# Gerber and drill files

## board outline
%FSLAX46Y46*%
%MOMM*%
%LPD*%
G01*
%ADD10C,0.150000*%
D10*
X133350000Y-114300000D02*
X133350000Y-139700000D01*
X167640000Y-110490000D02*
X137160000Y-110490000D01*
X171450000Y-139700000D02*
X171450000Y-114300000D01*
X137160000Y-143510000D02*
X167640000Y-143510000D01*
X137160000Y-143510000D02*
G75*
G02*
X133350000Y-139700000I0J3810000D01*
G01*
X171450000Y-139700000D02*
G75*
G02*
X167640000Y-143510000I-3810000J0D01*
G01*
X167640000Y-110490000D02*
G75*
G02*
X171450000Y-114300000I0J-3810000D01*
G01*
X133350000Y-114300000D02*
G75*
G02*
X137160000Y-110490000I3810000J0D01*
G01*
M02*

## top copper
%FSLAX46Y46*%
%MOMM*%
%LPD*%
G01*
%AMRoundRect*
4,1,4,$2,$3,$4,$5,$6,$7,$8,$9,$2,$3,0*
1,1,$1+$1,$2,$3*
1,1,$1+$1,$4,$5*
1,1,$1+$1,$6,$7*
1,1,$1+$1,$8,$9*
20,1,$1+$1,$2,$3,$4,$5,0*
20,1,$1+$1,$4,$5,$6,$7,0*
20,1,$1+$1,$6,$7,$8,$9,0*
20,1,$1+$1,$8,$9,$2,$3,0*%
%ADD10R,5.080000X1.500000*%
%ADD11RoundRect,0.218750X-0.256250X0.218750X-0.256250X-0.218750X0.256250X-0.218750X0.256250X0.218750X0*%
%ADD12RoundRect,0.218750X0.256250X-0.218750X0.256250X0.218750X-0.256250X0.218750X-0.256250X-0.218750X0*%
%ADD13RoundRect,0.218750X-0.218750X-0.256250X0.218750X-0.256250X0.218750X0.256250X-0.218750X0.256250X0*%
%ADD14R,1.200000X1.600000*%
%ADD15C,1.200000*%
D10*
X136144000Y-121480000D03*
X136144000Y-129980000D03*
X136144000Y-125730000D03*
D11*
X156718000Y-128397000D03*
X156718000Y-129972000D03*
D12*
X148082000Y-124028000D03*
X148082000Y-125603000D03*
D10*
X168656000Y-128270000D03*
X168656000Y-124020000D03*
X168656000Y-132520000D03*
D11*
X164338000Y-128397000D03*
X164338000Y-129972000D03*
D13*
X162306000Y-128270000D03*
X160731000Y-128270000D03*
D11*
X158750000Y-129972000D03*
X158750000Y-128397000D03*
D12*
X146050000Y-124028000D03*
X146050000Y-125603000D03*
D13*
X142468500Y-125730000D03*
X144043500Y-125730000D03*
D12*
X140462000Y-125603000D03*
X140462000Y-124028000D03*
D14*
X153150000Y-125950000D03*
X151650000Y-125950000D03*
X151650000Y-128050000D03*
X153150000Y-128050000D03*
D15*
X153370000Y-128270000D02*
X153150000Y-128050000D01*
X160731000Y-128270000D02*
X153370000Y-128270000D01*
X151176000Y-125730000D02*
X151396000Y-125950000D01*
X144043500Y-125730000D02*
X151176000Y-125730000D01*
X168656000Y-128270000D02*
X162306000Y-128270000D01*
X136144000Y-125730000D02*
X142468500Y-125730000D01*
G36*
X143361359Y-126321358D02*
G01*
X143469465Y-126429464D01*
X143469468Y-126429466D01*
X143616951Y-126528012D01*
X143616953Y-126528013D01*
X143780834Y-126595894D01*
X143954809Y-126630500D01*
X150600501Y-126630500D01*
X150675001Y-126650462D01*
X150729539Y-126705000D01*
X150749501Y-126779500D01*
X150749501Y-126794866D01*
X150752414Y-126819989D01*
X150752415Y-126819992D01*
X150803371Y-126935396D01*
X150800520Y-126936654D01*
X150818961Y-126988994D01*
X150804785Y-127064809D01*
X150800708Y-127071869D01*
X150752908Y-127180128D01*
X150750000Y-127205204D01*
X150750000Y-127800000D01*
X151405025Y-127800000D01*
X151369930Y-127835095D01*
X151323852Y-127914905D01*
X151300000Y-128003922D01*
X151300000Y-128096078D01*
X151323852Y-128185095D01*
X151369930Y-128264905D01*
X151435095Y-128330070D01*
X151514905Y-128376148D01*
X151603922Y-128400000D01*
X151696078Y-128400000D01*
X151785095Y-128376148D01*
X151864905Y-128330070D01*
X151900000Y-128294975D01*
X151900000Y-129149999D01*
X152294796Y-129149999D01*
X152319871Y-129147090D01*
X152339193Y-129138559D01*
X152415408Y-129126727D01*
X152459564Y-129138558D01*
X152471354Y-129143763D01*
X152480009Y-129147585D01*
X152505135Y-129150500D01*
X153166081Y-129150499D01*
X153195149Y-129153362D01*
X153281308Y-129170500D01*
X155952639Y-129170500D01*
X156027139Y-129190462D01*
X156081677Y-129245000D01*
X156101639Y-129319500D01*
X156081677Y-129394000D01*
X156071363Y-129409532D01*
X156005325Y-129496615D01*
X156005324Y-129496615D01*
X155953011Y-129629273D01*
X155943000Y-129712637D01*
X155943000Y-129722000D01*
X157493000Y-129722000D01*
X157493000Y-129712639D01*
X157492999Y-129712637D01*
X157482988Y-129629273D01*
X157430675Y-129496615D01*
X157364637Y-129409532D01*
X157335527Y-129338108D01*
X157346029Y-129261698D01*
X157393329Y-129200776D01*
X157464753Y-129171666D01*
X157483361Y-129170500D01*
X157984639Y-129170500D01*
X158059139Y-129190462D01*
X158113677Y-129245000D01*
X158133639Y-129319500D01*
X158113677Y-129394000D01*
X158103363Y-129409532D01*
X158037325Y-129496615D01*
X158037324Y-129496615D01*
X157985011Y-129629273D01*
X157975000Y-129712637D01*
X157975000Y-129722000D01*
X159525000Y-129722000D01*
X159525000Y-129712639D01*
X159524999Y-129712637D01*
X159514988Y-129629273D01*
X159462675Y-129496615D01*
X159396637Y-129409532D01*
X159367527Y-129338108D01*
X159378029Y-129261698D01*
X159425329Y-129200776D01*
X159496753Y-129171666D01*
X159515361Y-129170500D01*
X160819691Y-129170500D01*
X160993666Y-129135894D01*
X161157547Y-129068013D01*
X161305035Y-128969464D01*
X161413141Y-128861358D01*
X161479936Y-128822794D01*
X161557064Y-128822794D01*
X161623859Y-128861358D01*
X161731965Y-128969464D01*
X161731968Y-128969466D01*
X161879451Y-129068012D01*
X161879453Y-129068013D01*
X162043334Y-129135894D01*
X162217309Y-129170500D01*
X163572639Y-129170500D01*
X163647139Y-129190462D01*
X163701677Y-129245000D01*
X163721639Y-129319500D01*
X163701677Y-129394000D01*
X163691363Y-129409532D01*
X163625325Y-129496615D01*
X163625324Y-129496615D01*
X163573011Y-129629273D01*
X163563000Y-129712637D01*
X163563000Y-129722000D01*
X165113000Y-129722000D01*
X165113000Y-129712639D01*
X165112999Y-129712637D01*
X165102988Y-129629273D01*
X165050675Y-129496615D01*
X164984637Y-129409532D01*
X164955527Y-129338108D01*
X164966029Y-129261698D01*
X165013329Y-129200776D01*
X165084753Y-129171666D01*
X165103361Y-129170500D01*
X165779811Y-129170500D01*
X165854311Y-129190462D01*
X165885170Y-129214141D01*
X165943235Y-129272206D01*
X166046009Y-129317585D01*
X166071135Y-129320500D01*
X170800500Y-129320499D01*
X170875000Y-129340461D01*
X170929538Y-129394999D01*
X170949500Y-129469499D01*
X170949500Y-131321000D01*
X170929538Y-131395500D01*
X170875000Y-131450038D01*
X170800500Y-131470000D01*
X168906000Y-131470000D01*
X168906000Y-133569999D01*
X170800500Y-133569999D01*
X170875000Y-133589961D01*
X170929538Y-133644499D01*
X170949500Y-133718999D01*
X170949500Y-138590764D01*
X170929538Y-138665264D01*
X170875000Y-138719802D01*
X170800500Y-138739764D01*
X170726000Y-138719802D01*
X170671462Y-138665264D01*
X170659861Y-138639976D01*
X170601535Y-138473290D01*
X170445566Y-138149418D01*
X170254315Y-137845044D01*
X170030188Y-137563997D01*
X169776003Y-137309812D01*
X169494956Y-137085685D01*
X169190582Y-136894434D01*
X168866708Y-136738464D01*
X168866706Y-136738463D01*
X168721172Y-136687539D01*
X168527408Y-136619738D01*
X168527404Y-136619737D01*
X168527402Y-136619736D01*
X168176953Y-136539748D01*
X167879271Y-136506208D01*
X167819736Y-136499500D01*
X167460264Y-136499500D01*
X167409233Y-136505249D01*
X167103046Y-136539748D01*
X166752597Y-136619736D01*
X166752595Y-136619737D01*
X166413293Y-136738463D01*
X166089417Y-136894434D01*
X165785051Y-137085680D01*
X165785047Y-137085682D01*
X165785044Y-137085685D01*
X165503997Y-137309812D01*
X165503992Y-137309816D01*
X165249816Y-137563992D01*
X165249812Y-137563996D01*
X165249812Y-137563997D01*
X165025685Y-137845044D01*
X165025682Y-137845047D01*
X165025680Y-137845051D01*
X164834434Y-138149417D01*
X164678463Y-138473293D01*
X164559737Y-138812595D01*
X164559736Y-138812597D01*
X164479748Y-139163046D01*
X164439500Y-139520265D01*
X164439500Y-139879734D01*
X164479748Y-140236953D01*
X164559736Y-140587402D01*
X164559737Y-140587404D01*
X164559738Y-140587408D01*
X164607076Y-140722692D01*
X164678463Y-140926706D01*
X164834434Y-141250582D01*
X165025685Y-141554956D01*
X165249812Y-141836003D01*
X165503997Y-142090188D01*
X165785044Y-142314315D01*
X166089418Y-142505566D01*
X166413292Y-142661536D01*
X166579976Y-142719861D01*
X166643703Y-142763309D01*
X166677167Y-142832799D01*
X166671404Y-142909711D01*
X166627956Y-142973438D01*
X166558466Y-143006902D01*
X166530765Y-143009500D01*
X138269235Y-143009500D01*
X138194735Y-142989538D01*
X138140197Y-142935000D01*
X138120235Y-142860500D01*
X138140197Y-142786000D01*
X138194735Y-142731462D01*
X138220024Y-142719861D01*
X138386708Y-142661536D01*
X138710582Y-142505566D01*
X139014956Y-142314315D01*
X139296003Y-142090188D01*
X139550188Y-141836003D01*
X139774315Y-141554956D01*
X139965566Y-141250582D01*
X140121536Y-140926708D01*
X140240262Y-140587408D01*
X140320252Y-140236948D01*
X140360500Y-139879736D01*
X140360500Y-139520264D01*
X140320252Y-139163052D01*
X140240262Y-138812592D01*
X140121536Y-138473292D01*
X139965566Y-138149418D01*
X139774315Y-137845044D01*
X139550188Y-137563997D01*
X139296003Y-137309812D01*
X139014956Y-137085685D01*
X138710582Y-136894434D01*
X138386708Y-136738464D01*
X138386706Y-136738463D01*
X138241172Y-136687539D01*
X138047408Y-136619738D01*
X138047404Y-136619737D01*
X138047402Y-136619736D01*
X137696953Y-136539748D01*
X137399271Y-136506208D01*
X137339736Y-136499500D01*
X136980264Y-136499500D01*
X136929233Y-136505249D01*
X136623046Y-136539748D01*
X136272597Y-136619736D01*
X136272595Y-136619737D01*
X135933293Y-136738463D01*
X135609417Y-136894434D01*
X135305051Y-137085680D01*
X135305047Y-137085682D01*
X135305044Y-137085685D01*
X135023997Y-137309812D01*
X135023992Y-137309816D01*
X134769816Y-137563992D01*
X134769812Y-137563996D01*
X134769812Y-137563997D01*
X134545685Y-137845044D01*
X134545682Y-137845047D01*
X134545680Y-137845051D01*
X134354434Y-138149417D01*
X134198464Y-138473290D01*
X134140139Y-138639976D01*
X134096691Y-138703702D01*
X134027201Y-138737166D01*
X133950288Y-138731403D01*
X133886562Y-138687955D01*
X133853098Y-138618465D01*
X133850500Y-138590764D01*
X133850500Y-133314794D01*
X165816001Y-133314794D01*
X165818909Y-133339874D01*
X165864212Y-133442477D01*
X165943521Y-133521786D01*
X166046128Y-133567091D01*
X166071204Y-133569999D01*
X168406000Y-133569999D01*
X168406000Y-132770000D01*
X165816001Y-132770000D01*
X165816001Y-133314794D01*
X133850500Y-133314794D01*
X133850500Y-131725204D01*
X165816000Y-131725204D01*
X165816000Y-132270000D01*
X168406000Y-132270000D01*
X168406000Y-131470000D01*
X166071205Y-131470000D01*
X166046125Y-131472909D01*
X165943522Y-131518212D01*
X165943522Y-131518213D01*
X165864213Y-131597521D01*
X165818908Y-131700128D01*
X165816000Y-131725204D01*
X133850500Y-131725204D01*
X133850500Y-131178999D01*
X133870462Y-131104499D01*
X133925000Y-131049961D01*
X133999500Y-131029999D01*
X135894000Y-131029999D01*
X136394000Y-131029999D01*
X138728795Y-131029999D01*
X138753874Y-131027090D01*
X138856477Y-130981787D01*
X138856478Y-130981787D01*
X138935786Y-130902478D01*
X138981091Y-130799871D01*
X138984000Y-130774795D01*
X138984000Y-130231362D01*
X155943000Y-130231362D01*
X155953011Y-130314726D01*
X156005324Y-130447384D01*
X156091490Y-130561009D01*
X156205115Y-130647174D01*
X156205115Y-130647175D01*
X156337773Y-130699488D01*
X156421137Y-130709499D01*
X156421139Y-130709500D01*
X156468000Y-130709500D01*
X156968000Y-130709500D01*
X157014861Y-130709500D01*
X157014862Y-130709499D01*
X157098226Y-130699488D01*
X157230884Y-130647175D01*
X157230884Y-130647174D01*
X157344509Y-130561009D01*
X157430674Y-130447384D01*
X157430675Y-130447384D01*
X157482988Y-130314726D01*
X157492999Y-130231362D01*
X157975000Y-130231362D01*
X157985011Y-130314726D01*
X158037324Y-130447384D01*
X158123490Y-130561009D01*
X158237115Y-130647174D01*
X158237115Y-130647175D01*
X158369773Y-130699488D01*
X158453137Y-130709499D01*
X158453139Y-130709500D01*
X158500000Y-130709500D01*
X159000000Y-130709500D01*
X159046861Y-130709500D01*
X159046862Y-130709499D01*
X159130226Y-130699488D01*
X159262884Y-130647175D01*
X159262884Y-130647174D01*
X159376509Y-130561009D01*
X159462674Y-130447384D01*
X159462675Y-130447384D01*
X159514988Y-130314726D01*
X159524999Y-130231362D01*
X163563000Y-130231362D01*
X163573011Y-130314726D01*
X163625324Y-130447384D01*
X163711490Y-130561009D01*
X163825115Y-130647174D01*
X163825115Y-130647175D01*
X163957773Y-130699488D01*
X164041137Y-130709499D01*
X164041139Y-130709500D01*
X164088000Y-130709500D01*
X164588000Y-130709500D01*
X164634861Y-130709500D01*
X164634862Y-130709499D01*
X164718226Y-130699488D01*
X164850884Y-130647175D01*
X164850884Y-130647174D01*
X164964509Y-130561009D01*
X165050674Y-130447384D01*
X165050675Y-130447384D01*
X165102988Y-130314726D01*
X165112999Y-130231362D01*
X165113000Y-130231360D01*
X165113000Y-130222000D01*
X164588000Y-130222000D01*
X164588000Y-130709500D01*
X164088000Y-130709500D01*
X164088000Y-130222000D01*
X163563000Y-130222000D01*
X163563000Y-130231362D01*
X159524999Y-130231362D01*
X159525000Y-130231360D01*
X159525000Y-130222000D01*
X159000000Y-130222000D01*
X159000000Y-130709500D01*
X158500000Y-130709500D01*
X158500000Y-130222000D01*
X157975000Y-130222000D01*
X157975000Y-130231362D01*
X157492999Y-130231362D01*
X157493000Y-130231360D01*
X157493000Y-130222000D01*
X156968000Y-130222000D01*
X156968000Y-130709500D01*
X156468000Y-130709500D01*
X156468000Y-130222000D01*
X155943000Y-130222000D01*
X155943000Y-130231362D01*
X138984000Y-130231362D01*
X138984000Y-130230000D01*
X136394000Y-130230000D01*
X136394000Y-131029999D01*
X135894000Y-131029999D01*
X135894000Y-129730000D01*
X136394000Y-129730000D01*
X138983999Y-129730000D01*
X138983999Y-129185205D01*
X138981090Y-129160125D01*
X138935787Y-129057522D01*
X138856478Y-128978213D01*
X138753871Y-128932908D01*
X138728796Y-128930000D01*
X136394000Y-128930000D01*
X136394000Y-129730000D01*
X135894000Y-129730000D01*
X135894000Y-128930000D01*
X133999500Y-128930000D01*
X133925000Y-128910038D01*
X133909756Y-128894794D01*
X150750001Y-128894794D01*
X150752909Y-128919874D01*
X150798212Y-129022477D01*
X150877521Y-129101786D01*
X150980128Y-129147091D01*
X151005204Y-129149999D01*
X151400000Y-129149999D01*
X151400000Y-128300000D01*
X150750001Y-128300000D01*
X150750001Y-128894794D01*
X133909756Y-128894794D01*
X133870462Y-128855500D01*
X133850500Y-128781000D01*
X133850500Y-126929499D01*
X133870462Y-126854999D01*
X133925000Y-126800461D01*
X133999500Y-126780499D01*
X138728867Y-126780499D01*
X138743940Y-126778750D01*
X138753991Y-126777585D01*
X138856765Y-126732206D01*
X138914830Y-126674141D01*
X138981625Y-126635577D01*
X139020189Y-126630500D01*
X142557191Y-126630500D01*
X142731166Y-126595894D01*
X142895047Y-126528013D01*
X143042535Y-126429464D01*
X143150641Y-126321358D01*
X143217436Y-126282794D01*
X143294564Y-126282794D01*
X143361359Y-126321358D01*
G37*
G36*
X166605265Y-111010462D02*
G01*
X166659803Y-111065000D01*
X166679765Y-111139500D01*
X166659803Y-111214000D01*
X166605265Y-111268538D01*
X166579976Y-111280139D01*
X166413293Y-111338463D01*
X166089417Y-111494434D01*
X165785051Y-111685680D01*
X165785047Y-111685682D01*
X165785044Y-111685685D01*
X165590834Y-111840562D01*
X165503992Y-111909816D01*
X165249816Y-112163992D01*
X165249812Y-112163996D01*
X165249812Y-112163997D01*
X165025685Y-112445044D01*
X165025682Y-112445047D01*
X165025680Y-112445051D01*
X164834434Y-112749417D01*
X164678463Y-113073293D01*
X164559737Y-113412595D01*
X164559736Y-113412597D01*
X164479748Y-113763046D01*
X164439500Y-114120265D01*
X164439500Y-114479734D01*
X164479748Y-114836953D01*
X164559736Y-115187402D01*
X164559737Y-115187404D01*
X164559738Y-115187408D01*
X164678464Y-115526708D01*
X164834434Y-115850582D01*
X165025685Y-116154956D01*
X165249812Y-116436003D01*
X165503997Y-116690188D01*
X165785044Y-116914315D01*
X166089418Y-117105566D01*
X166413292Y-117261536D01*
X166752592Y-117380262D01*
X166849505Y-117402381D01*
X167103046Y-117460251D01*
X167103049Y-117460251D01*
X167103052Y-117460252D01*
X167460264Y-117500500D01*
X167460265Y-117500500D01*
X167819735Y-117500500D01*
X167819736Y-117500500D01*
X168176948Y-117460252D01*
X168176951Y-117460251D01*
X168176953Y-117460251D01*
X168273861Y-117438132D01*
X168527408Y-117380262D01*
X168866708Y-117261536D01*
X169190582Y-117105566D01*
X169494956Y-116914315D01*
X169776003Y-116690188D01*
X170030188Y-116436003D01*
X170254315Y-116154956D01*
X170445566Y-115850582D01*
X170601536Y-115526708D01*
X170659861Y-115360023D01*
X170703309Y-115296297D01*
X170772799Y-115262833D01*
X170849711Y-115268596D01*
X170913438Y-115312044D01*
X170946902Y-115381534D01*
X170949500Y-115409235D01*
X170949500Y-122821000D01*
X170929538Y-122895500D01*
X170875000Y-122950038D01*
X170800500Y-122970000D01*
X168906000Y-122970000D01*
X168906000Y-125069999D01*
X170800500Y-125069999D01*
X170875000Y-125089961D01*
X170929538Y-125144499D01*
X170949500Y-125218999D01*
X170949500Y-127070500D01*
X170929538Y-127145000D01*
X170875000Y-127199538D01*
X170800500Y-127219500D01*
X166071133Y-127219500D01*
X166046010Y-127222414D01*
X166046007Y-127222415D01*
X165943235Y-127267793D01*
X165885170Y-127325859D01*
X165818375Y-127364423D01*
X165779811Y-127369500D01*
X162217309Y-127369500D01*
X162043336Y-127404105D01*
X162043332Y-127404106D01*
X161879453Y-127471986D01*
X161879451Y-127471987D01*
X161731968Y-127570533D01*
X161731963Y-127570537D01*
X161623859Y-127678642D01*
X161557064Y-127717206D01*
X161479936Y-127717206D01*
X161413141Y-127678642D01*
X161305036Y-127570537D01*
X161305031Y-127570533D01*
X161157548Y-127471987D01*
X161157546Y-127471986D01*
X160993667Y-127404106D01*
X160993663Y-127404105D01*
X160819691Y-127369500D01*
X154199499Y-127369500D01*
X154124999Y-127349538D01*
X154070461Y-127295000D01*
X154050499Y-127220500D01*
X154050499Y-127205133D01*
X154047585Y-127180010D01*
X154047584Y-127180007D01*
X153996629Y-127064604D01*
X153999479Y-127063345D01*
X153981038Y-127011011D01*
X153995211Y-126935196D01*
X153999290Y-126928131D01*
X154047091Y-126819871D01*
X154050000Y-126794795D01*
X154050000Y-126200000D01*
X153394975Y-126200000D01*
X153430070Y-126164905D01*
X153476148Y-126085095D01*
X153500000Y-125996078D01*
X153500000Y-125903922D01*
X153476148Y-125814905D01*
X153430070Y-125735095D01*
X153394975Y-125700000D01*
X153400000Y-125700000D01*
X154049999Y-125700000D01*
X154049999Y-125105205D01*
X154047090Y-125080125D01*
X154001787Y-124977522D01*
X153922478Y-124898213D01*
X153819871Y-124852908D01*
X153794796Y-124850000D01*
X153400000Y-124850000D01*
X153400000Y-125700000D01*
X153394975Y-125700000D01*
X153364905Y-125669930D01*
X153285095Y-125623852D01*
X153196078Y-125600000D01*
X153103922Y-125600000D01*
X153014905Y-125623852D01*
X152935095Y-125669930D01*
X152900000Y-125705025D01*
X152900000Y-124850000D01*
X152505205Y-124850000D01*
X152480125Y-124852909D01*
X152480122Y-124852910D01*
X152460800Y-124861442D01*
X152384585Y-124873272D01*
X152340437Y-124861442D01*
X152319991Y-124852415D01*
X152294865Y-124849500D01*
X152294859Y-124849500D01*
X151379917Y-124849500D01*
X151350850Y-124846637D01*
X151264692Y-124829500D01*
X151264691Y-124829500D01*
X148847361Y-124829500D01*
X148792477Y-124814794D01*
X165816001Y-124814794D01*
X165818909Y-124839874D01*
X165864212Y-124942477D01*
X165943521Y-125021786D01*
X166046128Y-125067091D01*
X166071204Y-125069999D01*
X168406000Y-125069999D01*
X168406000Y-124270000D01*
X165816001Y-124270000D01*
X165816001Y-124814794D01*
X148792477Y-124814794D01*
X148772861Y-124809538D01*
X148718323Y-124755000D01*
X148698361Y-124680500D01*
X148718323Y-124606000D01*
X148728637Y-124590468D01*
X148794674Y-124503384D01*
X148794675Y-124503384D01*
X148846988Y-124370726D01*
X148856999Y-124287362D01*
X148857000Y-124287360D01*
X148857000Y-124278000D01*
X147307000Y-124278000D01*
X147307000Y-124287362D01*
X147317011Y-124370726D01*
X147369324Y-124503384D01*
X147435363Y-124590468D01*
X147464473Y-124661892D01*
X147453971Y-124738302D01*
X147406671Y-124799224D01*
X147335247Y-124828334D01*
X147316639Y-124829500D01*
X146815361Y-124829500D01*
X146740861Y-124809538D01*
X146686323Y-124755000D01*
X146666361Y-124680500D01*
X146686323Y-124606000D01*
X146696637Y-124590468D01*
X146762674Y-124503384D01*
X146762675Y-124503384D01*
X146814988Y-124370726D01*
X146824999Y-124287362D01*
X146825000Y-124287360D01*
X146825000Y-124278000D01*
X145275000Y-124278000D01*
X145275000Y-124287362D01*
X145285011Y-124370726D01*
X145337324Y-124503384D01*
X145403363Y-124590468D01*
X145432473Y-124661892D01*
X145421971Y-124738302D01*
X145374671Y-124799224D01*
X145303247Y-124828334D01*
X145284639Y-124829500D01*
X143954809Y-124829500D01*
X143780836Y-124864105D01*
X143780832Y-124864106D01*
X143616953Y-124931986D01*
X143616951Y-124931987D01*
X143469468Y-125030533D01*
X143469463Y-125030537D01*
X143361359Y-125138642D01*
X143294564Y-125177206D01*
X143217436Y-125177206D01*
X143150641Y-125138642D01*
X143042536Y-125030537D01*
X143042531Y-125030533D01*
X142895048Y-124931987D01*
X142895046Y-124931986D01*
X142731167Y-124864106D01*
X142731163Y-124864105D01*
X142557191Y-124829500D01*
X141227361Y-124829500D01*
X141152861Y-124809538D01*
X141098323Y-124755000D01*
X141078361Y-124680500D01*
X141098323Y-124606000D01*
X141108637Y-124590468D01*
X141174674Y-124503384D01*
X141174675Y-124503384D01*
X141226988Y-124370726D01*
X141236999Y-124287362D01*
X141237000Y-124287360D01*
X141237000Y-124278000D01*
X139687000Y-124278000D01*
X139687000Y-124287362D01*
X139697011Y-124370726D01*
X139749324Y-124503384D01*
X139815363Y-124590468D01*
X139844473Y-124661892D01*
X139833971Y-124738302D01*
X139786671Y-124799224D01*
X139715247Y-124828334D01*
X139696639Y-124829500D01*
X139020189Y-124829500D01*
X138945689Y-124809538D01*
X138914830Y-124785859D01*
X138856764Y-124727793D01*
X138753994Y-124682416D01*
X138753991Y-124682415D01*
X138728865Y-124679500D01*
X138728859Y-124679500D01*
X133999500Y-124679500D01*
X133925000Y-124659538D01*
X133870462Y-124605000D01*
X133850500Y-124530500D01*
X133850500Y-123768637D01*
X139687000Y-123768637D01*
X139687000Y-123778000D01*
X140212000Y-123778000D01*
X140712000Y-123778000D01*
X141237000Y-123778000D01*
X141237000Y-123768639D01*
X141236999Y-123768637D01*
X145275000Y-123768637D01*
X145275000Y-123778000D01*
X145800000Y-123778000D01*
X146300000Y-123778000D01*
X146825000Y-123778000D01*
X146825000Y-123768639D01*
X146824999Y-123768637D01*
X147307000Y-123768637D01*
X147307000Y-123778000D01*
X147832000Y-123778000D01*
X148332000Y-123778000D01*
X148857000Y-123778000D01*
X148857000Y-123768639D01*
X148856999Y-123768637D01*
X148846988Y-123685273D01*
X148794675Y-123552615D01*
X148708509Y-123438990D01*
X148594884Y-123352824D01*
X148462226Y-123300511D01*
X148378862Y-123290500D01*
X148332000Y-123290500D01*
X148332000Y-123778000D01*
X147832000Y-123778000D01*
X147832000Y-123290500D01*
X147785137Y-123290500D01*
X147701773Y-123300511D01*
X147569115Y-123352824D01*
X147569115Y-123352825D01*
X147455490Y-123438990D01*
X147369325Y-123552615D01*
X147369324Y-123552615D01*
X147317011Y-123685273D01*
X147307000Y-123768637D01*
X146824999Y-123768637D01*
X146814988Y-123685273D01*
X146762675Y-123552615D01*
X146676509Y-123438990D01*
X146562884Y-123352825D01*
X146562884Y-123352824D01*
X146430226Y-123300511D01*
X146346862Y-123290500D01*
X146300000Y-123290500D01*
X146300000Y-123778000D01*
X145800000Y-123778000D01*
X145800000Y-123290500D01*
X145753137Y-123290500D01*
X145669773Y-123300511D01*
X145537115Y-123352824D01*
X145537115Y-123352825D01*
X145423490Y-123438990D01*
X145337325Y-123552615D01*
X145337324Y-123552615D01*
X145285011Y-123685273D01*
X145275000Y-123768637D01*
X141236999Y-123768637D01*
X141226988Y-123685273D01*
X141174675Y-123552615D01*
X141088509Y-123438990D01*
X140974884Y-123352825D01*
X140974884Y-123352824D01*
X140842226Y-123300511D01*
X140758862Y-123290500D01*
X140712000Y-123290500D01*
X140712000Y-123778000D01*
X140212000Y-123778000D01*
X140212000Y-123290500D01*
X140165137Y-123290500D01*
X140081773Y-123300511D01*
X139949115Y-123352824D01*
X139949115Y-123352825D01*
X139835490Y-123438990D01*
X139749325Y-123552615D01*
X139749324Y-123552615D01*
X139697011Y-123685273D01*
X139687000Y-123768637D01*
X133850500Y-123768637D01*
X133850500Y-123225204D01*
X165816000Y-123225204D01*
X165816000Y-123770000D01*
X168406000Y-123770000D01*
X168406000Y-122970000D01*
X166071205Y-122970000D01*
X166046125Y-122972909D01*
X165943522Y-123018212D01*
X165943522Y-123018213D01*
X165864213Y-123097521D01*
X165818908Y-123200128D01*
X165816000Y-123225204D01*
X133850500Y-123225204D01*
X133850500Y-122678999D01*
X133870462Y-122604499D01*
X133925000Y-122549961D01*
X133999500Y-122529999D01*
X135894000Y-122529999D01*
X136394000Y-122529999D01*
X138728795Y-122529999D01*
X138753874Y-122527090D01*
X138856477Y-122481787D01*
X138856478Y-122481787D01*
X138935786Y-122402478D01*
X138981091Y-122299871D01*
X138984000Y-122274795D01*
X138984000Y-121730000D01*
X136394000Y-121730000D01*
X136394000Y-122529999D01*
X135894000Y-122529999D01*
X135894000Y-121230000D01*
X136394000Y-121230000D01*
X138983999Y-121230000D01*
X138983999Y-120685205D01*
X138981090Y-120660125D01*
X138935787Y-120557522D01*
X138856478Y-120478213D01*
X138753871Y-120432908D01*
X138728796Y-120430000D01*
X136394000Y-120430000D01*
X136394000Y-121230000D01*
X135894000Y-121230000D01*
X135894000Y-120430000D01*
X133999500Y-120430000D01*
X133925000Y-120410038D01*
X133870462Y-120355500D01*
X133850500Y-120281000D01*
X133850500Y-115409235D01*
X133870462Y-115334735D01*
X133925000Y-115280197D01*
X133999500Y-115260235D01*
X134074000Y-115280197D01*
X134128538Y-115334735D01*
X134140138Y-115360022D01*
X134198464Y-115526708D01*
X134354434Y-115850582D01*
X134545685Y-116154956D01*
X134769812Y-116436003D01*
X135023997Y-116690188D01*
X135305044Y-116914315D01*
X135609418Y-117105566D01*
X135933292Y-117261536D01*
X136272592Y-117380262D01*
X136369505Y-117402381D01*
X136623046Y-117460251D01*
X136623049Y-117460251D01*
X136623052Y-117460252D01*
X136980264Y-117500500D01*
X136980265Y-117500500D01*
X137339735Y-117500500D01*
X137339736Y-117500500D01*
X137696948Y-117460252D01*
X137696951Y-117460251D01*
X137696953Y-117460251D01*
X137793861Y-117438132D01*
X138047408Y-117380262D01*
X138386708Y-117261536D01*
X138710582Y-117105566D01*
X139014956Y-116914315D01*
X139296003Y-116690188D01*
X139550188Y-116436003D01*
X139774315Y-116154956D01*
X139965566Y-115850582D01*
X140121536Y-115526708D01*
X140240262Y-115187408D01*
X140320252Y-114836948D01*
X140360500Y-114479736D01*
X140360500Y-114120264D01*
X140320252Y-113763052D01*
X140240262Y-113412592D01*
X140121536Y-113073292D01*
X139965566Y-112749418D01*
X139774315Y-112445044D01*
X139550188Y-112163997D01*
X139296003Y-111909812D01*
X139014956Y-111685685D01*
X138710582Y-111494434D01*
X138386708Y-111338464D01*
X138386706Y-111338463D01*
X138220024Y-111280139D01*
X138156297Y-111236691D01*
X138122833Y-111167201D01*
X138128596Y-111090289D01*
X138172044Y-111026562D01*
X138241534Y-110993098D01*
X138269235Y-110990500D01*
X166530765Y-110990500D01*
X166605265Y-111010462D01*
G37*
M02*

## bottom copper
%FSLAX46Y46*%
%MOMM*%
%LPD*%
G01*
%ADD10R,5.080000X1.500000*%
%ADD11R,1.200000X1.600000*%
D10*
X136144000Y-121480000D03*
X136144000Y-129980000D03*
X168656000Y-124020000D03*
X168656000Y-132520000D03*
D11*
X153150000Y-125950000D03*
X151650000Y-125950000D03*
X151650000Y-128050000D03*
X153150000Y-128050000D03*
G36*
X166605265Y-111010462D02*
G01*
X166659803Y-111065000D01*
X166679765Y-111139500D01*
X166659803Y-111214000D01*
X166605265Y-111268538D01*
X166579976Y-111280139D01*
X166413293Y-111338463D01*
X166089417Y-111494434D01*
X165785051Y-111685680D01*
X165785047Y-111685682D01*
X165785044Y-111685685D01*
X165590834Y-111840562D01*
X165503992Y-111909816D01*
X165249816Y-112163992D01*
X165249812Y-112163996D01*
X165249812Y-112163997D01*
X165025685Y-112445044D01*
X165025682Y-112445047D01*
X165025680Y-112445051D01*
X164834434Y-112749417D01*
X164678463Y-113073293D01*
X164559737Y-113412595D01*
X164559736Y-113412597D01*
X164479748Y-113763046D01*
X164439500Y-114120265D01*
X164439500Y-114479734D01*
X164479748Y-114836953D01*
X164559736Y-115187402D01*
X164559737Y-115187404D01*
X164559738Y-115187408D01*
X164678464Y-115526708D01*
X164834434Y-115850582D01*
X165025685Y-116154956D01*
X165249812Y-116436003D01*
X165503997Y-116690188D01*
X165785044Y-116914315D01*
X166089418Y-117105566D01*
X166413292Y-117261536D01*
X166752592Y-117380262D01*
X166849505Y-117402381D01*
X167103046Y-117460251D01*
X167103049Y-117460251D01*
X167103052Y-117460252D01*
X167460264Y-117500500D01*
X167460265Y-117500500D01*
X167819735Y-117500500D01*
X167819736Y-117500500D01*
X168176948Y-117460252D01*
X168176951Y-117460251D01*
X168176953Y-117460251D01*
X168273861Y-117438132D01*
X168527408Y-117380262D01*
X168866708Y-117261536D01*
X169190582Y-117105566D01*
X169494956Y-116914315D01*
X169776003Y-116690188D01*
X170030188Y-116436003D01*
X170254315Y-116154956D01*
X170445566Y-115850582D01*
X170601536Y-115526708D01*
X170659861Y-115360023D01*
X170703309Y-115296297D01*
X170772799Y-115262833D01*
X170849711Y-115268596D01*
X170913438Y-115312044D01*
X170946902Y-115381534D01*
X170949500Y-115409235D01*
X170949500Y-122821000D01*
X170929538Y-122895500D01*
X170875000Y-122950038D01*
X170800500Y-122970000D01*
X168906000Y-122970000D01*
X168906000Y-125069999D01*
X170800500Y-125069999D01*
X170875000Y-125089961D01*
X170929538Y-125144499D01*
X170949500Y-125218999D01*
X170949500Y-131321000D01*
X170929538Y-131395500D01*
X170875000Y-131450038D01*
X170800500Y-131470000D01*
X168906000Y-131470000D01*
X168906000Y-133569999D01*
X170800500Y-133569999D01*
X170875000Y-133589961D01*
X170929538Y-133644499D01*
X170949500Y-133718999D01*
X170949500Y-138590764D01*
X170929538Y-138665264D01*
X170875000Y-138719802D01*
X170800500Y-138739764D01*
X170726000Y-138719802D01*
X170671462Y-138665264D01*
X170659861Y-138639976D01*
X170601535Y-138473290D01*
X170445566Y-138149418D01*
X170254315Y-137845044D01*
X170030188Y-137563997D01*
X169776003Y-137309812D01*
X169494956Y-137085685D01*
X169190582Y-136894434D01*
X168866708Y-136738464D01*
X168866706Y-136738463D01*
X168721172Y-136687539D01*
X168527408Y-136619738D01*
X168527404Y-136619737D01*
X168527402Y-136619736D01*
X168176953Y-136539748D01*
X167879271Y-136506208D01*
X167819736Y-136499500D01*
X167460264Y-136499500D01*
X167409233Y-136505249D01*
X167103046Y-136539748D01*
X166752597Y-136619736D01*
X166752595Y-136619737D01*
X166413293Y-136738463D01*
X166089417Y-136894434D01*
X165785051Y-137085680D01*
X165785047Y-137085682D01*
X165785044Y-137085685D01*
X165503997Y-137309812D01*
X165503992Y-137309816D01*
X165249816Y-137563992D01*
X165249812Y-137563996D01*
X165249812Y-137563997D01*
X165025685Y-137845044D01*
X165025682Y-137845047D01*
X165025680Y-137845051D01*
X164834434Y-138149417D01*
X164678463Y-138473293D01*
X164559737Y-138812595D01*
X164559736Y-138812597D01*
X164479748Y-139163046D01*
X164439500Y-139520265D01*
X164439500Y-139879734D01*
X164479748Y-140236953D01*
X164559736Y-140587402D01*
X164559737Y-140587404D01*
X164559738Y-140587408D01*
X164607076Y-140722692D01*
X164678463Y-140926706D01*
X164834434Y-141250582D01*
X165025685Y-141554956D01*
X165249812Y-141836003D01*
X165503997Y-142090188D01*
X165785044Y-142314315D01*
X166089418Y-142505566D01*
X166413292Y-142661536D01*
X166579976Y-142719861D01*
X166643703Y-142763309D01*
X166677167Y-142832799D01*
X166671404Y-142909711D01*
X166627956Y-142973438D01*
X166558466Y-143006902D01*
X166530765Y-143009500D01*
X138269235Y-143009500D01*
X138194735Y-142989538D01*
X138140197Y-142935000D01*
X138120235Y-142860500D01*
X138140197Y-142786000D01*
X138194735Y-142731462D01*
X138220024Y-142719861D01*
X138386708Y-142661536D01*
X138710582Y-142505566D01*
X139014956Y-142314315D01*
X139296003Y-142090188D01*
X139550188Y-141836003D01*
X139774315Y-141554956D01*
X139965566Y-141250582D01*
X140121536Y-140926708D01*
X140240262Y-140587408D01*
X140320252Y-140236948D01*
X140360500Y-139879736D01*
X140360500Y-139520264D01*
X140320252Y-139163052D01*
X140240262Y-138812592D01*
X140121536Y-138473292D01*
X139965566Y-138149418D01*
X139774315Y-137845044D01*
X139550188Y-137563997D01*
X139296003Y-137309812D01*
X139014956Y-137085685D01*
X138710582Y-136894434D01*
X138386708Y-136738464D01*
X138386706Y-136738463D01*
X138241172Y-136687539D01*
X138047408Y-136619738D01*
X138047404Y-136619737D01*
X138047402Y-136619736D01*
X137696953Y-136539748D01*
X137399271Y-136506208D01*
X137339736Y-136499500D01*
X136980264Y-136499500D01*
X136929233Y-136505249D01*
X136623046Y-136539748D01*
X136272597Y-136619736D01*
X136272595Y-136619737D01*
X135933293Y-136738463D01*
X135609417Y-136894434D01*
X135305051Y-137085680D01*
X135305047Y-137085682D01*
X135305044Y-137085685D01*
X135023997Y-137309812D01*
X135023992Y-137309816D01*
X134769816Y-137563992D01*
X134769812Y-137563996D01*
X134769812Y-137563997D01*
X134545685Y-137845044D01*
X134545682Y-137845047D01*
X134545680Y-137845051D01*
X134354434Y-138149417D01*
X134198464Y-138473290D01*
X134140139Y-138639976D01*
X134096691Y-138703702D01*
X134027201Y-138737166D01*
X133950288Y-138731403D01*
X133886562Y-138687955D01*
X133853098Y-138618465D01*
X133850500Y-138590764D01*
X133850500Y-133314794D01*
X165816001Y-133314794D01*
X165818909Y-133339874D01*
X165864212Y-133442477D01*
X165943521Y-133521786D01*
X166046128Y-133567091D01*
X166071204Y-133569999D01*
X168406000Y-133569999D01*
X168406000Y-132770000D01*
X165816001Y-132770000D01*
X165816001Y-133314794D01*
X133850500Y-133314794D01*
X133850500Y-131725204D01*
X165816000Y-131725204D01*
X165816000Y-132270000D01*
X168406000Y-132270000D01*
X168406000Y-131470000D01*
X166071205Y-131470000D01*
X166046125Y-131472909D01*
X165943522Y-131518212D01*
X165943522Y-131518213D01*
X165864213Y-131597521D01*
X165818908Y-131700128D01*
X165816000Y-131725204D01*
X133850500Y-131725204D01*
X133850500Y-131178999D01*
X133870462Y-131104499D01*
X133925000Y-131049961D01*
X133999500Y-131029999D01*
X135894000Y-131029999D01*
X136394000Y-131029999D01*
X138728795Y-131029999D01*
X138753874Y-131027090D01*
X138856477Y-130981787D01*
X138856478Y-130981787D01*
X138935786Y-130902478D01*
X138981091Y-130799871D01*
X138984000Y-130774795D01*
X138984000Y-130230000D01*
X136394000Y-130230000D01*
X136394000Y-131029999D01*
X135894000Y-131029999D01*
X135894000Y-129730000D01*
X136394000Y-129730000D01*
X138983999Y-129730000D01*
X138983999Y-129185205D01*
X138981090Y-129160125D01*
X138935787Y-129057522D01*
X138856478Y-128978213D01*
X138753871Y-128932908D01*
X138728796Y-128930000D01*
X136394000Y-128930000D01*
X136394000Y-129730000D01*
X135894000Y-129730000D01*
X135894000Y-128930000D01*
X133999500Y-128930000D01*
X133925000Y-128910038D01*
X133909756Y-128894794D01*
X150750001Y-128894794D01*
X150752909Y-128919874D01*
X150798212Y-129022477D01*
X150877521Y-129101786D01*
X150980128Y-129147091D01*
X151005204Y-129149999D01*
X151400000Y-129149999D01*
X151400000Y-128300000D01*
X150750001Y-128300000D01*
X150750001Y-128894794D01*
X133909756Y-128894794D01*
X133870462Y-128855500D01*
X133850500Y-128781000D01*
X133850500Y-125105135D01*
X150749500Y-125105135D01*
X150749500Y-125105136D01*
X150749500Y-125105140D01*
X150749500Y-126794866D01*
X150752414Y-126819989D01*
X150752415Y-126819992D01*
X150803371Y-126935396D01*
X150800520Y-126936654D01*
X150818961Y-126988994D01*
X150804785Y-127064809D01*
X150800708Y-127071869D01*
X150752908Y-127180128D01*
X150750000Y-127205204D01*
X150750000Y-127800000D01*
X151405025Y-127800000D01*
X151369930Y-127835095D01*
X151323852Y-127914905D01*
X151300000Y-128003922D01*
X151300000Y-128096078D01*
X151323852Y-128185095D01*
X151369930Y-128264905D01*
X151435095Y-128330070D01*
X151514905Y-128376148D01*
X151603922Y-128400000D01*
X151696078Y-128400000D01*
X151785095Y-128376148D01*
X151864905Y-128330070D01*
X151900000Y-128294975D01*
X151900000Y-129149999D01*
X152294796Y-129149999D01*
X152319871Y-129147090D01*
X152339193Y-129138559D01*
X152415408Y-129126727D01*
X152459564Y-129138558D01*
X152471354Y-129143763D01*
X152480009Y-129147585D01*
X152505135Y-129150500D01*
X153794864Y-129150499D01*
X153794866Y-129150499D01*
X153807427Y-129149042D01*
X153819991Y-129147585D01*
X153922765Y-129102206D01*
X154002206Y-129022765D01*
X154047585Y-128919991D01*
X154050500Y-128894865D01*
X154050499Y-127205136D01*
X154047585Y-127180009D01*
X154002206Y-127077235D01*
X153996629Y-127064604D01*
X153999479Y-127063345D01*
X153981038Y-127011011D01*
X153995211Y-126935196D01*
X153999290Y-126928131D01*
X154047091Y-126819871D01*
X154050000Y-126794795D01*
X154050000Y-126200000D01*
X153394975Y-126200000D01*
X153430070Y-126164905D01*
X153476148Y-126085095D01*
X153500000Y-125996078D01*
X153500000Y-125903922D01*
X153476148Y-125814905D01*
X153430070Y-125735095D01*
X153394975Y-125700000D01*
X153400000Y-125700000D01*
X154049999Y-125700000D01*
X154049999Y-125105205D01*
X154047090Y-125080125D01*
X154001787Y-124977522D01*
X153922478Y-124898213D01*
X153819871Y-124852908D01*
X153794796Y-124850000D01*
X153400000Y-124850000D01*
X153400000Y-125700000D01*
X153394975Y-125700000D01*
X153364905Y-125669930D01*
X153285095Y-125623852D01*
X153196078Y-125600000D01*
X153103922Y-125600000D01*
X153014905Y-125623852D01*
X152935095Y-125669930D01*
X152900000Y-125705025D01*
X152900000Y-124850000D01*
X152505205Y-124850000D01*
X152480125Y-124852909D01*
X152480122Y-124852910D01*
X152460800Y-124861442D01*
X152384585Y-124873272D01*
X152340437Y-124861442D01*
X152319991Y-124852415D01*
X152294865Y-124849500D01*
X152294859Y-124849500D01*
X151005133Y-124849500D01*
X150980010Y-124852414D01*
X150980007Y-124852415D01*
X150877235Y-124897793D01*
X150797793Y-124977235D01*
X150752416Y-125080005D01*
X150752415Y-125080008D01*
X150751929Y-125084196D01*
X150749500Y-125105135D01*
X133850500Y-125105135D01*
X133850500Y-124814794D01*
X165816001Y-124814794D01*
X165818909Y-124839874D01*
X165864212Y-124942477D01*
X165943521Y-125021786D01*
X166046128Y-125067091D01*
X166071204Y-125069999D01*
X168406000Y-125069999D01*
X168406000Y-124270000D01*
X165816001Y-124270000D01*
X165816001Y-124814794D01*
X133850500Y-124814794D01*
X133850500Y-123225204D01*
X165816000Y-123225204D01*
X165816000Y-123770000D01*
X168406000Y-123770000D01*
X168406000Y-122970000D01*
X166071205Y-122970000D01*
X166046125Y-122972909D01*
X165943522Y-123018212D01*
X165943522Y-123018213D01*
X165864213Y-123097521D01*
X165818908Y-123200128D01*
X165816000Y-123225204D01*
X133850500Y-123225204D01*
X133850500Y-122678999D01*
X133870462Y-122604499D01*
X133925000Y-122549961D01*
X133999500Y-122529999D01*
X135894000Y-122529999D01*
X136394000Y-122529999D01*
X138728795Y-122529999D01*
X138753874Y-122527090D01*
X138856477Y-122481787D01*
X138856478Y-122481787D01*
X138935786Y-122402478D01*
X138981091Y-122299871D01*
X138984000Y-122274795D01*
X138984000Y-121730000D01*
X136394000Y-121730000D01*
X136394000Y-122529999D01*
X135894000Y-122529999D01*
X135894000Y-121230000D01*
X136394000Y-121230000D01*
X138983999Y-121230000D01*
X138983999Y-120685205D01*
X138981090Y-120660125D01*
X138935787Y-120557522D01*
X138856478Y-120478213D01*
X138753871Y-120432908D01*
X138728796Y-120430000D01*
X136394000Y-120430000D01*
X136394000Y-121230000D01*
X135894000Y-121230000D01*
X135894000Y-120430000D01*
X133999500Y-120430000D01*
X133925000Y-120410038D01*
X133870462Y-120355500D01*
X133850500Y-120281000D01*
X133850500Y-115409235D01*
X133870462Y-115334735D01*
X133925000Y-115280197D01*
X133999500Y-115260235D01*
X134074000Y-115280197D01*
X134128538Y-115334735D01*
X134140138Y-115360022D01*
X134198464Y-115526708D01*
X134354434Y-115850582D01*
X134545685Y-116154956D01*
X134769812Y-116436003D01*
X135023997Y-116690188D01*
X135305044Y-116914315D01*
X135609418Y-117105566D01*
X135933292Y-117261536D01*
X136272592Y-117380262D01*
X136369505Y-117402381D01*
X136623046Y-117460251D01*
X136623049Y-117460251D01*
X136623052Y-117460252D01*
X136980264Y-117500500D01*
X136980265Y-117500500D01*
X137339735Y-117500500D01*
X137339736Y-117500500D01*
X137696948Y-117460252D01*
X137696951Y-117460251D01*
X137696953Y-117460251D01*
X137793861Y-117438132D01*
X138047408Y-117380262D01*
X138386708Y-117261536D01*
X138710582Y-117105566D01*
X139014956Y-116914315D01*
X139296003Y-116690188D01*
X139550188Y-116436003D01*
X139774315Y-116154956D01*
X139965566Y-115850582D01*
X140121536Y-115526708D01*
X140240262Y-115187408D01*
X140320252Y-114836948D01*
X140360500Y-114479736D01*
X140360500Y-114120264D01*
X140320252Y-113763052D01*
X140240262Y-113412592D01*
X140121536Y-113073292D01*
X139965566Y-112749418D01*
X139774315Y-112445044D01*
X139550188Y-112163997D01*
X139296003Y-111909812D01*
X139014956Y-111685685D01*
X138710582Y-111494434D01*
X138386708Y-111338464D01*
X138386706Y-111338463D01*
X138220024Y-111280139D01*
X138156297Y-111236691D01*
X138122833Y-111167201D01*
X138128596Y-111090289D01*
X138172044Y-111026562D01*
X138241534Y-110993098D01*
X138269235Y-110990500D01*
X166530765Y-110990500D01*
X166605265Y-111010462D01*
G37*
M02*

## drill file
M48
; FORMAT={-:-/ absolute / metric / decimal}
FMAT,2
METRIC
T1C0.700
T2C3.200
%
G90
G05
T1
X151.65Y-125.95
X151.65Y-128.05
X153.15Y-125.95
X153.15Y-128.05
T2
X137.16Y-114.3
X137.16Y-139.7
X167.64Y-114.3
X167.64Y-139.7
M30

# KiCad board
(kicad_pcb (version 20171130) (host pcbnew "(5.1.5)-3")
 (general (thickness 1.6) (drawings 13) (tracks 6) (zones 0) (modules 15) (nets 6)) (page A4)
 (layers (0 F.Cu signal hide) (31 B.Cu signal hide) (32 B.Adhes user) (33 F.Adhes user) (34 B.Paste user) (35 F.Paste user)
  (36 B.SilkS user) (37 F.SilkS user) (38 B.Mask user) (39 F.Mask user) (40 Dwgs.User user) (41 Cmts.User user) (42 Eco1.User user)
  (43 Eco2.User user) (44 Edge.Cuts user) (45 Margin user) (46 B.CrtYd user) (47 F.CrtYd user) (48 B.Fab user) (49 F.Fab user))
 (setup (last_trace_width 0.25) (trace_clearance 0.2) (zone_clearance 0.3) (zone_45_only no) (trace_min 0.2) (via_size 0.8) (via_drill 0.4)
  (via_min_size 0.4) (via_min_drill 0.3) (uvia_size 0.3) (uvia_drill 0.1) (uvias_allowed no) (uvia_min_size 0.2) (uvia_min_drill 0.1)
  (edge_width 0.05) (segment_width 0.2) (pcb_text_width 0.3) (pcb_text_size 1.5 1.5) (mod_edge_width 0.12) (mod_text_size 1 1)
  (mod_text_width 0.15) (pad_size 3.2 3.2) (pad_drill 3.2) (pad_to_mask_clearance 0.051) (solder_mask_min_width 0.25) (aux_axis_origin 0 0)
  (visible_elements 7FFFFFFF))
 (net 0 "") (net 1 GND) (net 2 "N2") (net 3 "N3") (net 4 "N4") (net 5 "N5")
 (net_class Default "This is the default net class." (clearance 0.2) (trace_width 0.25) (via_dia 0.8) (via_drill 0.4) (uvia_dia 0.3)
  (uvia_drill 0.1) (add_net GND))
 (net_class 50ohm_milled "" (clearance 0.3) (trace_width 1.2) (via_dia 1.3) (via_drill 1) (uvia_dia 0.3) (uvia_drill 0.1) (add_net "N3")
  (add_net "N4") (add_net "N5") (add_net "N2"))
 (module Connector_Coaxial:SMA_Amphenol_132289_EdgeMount (layer F.Cu) (at 136.144 125.73 180)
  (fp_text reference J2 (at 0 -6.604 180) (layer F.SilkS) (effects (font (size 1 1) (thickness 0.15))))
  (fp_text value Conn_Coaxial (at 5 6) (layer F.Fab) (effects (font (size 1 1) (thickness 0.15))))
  (pad 2 smd rect (at 0 4.25 270) (size 1.5 5.08) (layers B.Cu B.Paste B.Mask) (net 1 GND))
  (pad 2 smd rect (at 0 -4.25 270) (size 1.5 5.08) (layers B.Cu B.Paste B.Mask) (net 1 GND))
  (pad 2 smd rect (at 0 4.25 270) (size 1.5 5.08) (layers F.Cu F.Paste F.Mask) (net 1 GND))
  (pad 2 smd rect (at 0 -4.25 270) (size 1.5 5.08) (layers F.Cu F.Paste F.Mask) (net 1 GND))
  (pad 1 smd rect (at 0 0 270) (size 1.5 5.08) (layers F.Cu F.Paste F.Mask) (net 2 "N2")))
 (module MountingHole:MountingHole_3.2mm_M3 (layer F.Cu) (at 137.16 139.7)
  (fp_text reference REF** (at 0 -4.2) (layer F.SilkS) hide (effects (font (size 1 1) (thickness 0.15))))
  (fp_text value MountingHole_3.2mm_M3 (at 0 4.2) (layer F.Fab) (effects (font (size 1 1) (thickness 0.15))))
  (pad "" np_thru_hole circle (at 0 0) (size 3.2 3.2) (drill 3.2) (layers *.Cu *.Mask) (clearance 1.6)))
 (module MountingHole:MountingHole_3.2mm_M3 (layer F.Cu) (at 167.64 139.7)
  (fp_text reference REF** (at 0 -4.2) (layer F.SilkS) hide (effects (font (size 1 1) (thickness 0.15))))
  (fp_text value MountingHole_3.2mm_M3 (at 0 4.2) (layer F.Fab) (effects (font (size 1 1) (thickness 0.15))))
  (pad "" np_thru_hole circle (at 0 0) (size 3.2 3.2) (drill 3.2) (layers *.Cu *.Mask) (clearance 1.6)))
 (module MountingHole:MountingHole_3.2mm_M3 (layer F.Cu) (at 167.64 114.3)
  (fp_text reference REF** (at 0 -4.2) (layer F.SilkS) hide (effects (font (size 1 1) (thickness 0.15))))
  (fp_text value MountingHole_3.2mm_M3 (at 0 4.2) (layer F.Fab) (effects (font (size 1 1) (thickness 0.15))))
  (pad "" np_thru_hole circle (at 0 0) (size 3.2 3.2) (drill 3.2) (layers *.Cu *.Mask) (clearance 1.6)))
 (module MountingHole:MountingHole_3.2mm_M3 (layer F.Cu) (at 137.16 114.3)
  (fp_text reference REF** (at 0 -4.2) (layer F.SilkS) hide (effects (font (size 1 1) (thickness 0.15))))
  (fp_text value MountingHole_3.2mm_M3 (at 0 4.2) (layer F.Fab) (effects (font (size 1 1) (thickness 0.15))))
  (pad "" np_thru_hole circle (at 0 0) (size 3.2 3.2) (drill 3.2) (layers *.Cu *.Mask) (clearance 1.6)))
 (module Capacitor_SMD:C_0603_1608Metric (layer F.Cu) (at 156.718 129.1845 270)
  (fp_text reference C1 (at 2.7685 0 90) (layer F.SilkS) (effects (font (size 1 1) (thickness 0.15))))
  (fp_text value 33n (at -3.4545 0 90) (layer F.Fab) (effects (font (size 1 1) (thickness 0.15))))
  (pad 1 smd roundrect (at -0.7875 0 270) (size 0.875 0.95) (layers F.Cu F.Paste F.Mask) (roundrect_rratio 0.25) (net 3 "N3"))
  (pad 2 smd roundrect (at 0.7875 0 270) (size 0.875 0.95) (layers F.Cu F.Paste F.Mask) (roundrect_rratio 0.25) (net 1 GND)))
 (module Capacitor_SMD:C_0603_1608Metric (layer F.Cu) (at 148.082 124.8155 90)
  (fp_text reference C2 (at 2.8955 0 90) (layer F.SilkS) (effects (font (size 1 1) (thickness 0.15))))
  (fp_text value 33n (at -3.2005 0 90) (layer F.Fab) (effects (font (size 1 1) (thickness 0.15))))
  (pad 2 smd roundrect (at 0.7875 0 90) (size 0.875 0.95) (layers F.Cu F.Paste F.Mask) (roundrect_rratio 0.25) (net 1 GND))
  (pad 1 smd roundrect (at -0.7875 0 90) (size 0.875 0.95) (layers F.Cu F.Paste F.Mask) (roundrect_rratio 0.25) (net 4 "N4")))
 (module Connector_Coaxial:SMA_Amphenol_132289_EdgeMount (layer F.Cu) (at 168.656 128.27)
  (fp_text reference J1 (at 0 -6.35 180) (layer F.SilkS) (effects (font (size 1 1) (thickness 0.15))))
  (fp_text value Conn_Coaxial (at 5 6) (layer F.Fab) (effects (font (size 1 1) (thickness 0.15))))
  (pad 1 smd rect (at 0 0 90) (size 1.5 5.08) (layers F.Cu F.Paste F.Mask) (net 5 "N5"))
  (pad 2 smd rect (at 0 -4.25 90) (size 1.5 5.08) (layers F.Cu F.Paste F.Mask) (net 1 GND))
  (pad 2 smd rect (at 0 4.25 90) (size 1.5 5.08) (layers F.Cu F.Paste F.Mask) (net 1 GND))
  (pad 2 smd rect (at 0 -4.25 90) (size 1.5 5.08) (layers B.Cu B.Paste B.Mask) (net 1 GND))
  (pad 2 smd rect (at 0 4.25 90) (size 1.5 5.08) (layers B.Cu B.Paste B.Mask) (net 1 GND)))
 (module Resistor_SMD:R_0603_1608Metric (layer F.Cu) (at 164.338 129.1845 270)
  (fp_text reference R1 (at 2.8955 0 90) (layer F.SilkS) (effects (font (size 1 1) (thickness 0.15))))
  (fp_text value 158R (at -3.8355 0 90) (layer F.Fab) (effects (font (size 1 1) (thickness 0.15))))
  (pad 1 smd roundrect (at -0.7875 0 270) (size 0.875 0.95) (layers F.Cu F.Paste F.Mask) (roundrect_rratio 0.25) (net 5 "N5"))
  (pad 2 smd roundrect (at 0.7875 0 270) (size 0.875 0.95) (layers F.Cu F.Paste F.Mask) (roundrect_rratio 0.25) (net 1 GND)))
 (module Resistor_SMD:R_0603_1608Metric (layer F.Cu) (at 161.5185 128.27)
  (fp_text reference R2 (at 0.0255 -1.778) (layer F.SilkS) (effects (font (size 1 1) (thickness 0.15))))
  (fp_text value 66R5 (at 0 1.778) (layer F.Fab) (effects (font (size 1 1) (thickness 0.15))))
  (pad 2 smd roundrect (at 0.7875 0) (size 0.875 0.95) (layers F.Cu F.Paste F.Mask) (roundrect_rratio 0.25) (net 5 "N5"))
  (pad 1 smd roundrect (at -0.7875 0) (size 0.875 0.95) (layers F.Cu F.Paste F.Mask) (roundrect_rratio 0.25) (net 3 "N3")))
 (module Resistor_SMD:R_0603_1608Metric (layer F.Cu) (at 158.75 129.1845 270)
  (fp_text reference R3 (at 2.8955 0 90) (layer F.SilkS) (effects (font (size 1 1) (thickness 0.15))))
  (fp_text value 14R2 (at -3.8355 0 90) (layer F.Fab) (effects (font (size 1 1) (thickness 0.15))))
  (pad 2 smd roundrect (at 0.7875 0 270) (size 0.875 0.95) (layers F.Cu F.Paste F.Mask) (roundrect_rratio 0.25) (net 1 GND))
  (pad 1 smd roundrect (at -0.7875 0 270) (size 0.875 0.95) (layers F.Cu F.Paste F.Mask) (roundrect_rratio 0.25) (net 3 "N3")))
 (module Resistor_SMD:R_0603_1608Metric (layer F.Cu) (at 146.05 124.8155 90)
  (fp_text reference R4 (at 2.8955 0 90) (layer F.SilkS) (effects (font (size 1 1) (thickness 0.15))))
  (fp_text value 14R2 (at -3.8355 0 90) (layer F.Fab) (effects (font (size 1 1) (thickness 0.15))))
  (pad 2 smd roundrect (at 0.7875 0 90) (size 0.875 0.95) (layers F.Cu F.Paste F.Mask) (roundrect_rratio 0.25) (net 1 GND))
  (pad 1 smd roundrect (at -0.7875 0 90) (size 0.875 0.95) (layers F.Cu F.Paste F.Mask) (roundrect_rratio 0.25) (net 4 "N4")))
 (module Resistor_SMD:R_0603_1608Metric (layer F.Cu) (at 143.256 125.73)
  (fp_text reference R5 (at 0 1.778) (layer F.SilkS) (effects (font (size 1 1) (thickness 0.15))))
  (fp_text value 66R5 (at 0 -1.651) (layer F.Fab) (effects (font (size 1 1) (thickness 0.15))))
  (pad 1 smd roundrect (at -0.7875 0) (size 0.875 0.95) (layers F.Cu F.Paste F.Mask) (roundrect_rratio 0.25) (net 2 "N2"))
  (pad 2 smd roundrect (at 0.7875 0) (size 0.875 0.95) (layers F.Cu F.Paste F.Mask) (roundrect_rratio 0.25) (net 4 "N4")))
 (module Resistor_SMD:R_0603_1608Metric (layer F.Cu) (at 140.462 124.8155 90)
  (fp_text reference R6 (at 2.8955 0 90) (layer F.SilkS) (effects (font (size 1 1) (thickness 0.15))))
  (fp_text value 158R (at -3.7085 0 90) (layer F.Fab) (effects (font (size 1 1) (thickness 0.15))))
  (pad 1 smd roundrect (at -0.7875 0 90) (size 0.875 0.95) (layers F.Cu F.Paste F.Mask) (roundrect_rratio 0.25) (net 2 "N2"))
  (pad 2 smd roundrect (at 0.7875 0 90) (size 0.875 0.95) (layers F.Cu F.Paste F.Mask) (roundrect_rratio 0.25) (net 1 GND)))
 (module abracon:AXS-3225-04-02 (layer F.Cu) (at 152.4 127 90)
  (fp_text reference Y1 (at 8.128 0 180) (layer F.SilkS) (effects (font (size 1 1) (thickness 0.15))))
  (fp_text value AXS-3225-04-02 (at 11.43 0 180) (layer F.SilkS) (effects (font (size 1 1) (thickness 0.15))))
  (pad 4 thru_hole rect (at 1.05 0.75 90) (size 1.6 1.2) (drill 0.7) (layers *.Cu *.Mask) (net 1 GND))
  (pad 3 thru_hole rect (at 1.05 -0.75 90) (size 1.6 1.2) (drill 0.7) (layers *.Cu *.Mask) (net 4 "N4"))
  (pad 2 thru_hole rect (at -1.05 -0.75 90) (size 1.6 1.2) (drill 0.7) (layers *.Cu *.Mask) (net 1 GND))
  (pad 1 thru_hole rect (at -1.05 0.75 90) (size 1.6 1.2) (drill 0.7) (layers *.Cu *.Mask) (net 3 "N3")))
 (gr_line (start 133.35 114.3) (end 133.35 139.7) (layer Edge.Cuts) (width 0.15))
 (gr_line (start 167.64 110.49) (end 137.16 110.49) (layer Edge.Cuts) (width 0.15))
 (gr_line (start 171.45 139.7) (end 171.45 114.3) (layer Edge.Cuts) (width 0.15))
 (gr_line (start 137.16 143.51) (end 167.64 143.51) (layer Edge.Cuts) (width 0.15))
 (gr_arc (start 137.16 139.7) (end 133.35 139.7) (angle -90) (layer Edge.Cuts) (width 0.15))
 (gr_arc (start 167.64 139.7) (end 167.64 143.51) (angle -90) (layer Edge.Cuts) (width 0.15))
 (gr_arc (start 167.64 114.3) (end 171.45 114.3) (angle -90) (layer Edge.Cuts) (width 0.15))
 (gr_arc (start 137.16 114.3) (end 137.16 110.49) (angle -90) (layer Edge.Cuts) (width 0.15))
 (segment (start 153.37 128.27) (end 153.15 128.05) (width 1.2) (layer F.Cu) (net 3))
 (segment (start 160.731 128.27) (end 153.37 128.27) (width 1.2) (layer F.Cu) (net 3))
 (segment (start 151.176 125.73) (end 151.396 125.95) (width 1.2) (layer F.Cu) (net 4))
 (segment (start 144.0435 125.73) (end 151.176 125.73) (width 1.2) (layer F.Cu) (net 4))
 (segment (start 168.656 128.27) (end 162.306 128.27) (width 1.2) (layer F.Cu) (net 5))
 (segment (start 136.144 125.73) (end 142.4685 125.73) (width 1.2) (layer F.Cu) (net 2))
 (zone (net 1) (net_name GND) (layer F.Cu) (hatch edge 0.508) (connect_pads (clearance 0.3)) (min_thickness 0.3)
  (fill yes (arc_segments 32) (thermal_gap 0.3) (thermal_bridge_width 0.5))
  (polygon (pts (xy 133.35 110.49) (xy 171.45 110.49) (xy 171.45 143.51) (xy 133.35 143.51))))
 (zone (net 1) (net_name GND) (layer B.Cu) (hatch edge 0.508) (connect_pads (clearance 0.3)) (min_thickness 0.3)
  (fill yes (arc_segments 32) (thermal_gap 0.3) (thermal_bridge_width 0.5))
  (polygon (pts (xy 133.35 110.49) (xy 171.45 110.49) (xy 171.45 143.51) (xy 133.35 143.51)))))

